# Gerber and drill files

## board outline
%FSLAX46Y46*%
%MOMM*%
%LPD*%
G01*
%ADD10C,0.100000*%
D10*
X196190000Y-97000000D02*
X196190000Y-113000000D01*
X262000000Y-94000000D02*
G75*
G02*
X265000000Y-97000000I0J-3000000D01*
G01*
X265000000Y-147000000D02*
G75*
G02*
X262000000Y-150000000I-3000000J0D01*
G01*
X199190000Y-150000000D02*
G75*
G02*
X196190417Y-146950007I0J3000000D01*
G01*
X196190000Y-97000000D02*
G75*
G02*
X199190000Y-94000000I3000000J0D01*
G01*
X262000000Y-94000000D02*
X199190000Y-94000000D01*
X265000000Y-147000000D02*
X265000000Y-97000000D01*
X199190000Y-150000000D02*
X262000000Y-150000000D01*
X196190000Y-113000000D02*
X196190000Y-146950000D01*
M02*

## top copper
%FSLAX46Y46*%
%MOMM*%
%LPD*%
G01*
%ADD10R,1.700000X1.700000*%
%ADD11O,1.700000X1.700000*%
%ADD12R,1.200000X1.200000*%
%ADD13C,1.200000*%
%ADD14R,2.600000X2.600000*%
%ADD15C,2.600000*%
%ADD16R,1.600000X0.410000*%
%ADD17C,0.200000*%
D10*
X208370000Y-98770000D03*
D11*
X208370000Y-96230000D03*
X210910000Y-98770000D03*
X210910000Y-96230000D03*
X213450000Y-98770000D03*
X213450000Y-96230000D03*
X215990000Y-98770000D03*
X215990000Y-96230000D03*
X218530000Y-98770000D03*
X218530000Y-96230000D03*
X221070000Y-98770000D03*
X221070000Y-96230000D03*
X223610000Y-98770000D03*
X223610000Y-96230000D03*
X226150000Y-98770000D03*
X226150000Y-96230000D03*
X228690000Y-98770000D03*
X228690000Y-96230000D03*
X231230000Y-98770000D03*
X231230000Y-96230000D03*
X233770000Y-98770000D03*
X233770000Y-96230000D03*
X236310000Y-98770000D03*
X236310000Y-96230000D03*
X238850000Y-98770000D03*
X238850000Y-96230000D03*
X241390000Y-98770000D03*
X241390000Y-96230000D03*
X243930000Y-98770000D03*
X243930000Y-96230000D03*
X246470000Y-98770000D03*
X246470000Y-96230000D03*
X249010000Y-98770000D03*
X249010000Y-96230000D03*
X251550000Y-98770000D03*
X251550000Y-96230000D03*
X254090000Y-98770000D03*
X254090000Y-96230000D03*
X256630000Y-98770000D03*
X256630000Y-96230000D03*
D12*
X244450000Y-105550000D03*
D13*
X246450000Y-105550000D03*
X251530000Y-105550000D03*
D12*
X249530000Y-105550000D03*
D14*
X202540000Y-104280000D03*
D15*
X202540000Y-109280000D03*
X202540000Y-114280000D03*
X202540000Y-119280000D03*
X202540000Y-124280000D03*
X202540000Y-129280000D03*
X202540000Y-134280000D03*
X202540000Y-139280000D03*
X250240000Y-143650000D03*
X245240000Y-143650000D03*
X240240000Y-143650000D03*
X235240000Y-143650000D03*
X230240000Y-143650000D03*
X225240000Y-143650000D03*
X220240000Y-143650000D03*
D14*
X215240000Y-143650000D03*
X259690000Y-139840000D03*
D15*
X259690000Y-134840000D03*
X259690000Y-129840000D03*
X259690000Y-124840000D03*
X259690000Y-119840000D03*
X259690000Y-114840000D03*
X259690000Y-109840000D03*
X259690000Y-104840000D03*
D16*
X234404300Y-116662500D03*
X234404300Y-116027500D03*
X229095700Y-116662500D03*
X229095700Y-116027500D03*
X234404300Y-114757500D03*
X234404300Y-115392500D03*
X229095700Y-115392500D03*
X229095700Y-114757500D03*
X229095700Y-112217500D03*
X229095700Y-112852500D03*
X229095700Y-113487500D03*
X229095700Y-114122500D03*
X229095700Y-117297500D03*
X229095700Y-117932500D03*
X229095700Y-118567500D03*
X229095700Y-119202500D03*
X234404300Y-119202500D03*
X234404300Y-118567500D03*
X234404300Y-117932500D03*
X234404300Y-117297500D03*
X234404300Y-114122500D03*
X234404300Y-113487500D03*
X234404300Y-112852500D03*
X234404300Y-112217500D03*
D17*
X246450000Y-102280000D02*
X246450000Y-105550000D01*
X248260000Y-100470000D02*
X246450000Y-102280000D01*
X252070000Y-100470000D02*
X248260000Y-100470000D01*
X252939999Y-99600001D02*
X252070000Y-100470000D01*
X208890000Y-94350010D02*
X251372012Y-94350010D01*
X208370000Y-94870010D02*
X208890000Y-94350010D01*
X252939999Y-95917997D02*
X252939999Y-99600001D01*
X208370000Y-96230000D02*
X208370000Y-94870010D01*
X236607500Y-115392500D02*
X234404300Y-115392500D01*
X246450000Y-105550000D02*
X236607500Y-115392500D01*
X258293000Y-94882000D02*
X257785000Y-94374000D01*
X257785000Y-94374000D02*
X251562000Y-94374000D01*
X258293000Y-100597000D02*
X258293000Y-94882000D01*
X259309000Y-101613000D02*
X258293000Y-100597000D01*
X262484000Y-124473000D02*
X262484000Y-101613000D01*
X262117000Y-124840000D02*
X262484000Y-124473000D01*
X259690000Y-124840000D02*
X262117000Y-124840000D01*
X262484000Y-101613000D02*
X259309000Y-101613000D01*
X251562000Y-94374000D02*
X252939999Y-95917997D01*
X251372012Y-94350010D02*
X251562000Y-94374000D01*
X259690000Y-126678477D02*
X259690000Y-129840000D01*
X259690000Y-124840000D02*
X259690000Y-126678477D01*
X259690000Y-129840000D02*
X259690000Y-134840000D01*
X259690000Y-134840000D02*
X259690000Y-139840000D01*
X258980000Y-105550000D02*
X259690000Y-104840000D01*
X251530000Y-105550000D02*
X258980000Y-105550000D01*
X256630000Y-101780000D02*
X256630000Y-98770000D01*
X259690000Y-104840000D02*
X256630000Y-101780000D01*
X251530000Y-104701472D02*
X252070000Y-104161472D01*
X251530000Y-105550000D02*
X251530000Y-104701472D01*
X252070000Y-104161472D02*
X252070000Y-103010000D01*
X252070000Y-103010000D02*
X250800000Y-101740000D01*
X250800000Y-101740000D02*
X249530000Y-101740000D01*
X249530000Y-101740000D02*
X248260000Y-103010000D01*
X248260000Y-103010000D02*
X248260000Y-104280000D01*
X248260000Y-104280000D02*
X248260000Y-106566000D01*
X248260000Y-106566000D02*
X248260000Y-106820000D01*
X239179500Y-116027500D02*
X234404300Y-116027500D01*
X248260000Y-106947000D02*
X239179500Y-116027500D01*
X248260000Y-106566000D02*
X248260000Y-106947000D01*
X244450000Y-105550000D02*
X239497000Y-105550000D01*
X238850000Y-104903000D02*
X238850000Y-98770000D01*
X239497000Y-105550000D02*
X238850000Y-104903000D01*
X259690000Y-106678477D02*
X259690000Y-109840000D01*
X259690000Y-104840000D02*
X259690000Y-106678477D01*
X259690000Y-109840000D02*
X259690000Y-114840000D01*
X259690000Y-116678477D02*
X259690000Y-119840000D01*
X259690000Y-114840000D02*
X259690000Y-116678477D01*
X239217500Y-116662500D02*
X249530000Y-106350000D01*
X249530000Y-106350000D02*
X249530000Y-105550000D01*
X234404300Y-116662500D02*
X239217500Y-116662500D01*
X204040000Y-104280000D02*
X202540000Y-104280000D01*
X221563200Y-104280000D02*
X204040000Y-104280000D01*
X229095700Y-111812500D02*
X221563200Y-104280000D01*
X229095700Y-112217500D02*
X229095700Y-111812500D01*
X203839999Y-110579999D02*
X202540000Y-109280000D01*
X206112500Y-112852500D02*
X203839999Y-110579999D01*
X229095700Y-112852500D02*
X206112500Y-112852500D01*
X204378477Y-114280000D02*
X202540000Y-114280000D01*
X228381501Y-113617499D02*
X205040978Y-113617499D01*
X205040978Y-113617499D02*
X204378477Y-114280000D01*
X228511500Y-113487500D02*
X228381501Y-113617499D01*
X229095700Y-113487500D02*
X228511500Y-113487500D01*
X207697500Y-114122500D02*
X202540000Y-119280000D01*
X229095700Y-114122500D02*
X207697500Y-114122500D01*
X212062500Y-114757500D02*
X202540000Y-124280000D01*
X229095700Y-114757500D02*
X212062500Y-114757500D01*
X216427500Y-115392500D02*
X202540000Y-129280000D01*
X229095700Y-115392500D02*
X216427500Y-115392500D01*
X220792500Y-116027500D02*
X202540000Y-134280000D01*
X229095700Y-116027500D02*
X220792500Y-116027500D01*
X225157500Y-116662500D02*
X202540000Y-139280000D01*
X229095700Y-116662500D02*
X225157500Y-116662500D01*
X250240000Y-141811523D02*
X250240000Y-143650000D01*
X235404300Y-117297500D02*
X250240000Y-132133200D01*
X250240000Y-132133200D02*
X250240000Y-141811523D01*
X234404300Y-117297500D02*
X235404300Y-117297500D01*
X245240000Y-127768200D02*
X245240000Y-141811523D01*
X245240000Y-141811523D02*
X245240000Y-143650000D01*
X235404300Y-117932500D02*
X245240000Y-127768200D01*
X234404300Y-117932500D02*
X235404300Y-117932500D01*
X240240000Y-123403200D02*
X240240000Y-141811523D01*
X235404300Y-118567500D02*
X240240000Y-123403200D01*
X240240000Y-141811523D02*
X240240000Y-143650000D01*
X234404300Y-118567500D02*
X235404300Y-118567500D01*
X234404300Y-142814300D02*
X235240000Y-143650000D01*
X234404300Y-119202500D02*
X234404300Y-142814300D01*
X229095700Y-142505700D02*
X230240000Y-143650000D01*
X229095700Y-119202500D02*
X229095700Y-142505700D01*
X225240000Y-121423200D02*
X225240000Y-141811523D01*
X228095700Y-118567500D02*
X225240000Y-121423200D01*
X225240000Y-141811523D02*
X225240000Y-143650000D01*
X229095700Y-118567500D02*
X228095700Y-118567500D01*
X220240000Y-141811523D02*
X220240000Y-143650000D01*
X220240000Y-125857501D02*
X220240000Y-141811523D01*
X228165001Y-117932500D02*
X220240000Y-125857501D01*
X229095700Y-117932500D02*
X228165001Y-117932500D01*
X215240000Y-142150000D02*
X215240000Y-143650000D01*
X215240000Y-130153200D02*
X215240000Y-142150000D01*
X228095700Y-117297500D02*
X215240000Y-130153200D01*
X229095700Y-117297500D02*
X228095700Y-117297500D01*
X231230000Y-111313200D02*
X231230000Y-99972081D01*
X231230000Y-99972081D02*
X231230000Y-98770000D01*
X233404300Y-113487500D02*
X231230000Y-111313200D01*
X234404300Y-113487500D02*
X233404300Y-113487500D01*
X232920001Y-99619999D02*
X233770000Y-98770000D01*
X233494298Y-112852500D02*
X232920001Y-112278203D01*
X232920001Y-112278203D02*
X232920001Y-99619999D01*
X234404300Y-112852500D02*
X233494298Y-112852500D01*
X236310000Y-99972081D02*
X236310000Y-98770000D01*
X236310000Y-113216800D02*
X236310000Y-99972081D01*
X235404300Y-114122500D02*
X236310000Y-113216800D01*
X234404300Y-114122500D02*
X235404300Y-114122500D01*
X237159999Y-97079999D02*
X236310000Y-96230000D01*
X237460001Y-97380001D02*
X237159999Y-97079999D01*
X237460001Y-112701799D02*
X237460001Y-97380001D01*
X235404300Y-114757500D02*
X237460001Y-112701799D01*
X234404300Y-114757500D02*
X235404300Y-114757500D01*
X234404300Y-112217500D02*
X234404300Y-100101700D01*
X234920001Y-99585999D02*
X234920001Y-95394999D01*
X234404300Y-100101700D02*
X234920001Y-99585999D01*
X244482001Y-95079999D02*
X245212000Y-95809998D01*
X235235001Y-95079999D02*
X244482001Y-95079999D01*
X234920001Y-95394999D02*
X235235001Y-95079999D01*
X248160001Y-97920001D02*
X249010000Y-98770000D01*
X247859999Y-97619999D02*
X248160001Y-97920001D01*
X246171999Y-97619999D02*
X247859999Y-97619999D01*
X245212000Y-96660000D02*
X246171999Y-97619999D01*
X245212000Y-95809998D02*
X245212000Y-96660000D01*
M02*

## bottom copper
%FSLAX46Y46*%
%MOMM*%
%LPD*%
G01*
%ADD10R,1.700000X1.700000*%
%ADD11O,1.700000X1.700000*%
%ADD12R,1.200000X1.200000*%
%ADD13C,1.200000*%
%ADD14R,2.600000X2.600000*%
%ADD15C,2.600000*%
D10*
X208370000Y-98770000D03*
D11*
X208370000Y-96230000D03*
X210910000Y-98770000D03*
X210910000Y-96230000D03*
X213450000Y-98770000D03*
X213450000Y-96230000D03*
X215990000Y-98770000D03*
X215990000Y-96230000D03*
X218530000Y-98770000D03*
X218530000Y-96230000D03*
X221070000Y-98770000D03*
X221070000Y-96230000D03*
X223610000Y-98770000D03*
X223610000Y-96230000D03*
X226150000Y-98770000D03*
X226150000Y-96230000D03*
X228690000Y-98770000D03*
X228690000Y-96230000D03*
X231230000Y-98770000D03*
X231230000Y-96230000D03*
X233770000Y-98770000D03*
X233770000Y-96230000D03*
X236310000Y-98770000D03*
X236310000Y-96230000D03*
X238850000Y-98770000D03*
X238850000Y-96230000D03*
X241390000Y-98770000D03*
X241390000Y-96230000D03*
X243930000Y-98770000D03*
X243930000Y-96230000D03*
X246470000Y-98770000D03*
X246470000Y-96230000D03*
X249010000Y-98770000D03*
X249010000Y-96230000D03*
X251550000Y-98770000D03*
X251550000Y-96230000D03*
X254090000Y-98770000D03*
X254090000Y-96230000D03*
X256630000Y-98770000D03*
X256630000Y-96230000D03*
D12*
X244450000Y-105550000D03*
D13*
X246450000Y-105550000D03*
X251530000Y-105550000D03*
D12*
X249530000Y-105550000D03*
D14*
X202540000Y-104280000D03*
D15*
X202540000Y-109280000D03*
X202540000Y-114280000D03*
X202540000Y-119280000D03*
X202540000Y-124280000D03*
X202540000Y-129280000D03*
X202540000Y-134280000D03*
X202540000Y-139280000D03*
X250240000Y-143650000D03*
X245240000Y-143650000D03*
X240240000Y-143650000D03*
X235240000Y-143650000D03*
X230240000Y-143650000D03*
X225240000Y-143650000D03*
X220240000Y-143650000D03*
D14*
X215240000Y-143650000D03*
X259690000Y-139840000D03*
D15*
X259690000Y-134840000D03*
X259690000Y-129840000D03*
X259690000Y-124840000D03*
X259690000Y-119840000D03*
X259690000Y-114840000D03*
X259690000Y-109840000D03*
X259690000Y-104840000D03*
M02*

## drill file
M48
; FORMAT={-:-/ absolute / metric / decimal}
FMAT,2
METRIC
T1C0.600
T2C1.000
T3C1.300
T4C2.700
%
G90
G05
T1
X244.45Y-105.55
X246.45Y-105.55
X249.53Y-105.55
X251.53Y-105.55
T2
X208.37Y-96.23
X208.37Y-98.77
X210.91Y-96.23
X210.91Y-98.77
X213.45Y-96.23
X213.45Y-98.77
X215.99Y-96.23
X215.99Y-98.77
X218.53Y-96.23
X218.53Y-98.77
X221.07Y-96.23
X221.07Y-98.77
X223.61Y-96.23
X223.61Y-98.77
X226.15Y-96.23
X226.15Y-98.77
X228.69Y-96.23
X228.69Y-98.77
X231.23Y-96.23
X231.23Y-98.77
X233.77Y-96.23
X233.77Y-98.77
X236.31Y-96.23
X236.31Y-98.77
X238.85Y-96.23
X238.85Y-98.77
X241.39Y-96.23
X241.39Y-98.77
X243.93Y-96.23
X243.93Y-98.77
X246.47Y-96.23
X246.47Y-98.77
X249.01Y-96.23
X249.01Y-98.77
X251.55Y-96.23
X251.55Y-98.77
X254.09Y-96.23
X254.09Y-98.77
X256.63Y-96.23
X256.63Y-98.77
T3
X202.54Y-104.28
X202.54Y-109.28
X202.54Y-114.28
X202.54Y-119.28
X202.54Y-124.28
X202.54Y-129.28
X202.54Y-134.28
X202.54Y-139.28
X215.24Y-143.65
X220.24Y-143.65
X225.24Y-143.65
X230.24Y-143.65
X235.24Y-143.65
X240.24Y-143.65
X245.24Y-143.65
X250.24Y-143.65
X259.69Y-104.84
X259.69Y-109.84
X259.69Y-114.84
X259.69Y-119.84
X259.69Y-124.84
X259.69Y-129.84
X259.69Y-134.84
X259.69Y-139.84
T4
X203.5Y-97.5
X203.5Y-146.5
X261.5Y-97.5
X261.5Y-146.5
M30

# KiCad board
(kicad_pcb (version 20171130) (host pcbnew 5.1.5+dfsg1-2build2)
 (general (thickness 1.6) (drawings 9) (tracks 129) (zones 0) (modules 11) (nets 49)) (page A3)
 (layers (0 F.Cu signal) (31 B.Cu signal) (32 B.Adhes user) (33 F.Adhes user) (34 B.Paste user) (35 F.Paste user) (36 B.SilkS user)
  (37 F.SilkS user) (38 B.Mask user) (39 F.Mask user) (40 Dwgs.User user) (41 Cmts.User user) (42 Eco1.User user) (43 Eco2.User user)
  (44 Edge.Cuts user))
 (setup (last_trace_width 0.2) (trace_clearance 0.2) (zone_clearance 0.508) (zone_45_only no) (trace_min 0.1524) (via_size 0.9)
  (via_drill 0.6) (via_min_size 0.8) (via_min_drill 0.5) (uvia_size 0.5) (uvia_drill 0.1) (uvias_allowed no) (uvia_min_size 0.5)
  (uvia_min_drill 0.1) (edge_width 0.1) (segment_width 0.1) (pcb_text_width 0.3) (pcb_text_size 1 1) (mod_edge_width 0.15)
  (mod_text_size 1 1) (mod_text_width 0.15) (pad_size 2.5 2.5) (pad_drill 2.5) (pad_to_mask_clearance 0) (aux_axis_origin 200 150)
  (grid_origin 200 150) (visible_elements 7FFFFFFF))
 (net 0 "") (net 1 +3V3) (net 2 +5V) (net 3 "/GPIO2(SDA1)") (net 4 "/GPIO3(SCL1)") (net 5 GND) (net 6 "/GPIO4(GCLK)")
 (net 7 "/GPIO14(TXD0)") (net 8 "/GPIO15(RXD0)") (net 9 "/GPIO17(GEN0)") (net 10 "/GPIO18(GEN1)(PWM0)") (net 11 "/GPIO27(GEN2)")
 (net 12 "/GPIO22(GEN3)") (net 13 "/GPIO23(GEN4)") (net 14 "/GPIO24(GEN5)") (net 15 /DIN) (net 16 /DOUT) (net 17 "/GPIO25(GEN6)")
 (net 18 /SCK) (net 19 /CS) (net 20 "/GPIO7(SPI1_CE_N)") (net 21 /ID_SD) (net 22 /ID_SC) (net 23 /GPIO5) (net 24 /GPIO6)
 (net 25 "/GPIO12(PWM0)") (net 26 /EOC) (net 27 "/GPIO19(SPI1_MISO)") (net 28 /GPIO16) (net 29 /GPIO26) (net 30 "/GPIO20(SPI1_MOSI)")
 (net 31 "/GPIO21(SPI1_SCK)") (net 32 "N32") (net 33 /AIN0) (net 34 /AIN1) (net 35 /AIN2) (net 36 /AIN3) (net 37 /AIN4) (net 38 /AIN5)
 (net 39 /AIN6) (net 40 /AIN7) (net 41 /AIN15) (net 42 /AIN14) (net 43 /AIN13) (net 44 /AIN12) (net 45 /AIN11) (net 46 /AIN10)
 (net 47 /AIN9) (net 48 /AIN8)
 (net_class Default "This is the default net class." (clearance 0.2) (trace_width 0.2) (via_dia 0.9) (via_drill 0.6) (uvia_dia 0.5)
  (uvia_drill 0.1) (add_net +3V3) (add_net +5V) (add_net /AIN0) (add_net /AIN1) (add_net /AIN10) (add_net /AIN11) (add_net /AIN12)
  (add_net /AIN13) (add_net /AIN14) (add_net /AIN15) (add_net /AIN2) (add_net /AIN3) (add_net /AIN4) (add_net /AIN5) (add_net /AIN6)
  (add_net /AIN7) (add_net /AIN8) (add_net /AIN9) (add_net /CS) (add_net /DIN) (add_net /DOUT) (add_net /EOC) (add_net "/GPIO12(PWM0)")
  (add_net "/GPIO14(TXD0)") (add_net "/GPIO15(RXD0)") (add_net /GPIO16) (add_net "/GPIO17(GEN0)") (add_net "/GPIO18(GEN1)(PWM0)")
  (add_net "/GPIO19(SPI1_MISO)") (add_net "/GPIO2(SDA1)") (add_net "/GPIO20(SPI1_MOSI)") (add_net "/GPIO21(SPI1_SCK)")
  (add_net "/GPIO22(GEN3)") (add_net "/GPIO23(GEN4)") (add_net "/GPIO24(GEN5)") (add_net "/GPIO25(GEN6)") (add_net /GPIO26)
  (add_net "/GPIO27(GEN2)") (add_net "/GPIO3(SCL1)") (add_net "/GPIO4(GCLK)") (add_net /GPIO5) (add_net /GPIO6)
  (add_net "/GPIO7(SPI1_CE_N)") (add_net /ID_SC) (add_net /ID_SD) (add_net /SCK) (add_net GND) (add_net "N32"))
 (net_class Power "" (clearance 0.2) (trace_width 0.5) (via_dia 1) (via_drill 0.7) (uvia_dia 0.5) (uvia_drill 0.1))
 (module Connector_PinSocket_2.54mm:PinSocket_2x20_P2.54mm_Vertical (layer B.Cu) (at 208.37 98.77 270)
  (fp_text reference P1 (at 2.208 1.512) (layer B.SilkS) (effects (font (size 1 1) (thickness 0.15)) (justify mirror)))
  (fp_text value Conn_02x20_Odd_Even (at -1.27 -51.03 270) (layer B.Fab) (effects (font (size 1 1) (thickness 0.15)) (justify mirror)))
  (pad 1 thru_hole rect (at 0 0 270) (size 1.7 1.7) (drill 1) (layers *.Cu *.Mask) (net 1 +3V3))
  (pad 2 thru_hole oval (at -2.54 0 270) (size 1.7 1.7) (drill 1) (layers *.Cu *.Mask) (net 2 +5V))
  (pad 3 thru_hole oval (at 0 -2.54 270) (size 1.7 1.7) (drill 1) (layers *.Cu *.Mask) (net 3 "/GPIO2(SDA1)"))
  (pad 4 thru_hole oval (at -2.54 -2.54 270) (size 1.7 1.7) (drill 1) (layers *.Cu *.Mask) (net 2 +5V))
  (pad 5 thru_hole oval (at 0 -5.08 270) (size 1.7 1.7) (drill 1) (layers *.Cu *.Mask) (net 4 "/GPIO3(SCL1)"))
  (pad 6 thru_hole oval (at -2.54 -5.08 270) (size 1.7 1.7) (drill 1) (layers *.Cu *.Mask) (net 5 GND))
  (pad 7 thru_hole oval (at 0 -7.62 270) (size 1.7 1.7) (drill 1) (layers *.Cu *.Mask) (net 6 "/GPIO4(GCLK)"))
  (pad 8 thru_hole oval (at -2.54 -7.62 270) (size 1.7 1.7) (drill 1) (layers *.Cu *.Mask) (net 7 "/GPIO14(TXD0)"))
  (pad 9 thru_hole oval (at 0 -10.16 270) (size 1.7 1.7) (drill 1) (layers *.Cu *.Mask) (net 5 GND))
  (pad 10 thru_hole oval (at -2.54 -10.16 270) (size 1.7 1.7) (drill 1) (layers *.Cu *.Mask) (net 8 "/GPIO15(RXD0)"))
  (pad 11 thru_hole oval (at 0 -12.7 270) (size 1.7 1.7) (drill 1) (layers *.Cu *.Mask) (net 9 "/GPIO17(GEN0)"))
  (pad 12 thru_hole oval (at -2.54 -12.7 270) (size 1.7 1.7) (drill 1) (layers *.Cu *.Mask) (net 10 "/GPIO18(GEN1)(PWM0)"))
  (pad 13 thru_hole oval (at 0 -15.24 270) (size 1.7 1.7) (drill 1) (layers *.Cu *.Mask) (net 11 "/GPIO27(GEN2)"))
  (pad 14 thru_hole oval (at -2.54 -15.24 270) (size 1.7 1.7) (drill 1) (layers *.Cu *.Mask) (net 5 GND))
  (pad 15 thru_hole oval (at 0 -17.78 270) (size 1.7 1.7) (drill 1) (layers *.Cu *.Mask) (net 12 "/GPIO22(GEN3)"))
  (pad 16 thru_hole oval (at -2.54 -17.78 270) (size 1.7 1.7) (drill 1) (layers *.Cu *.Mask) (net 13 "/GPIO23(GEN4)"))
  (pad 17 thru_hole oval (at 0 -20.32 270) (size 1.7 1.7) (drill 1) (layers *.Cu *.Mask) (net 1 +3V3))
  (pad 18 thru_hole oval (at -2.54 -20.32 270) (size 1.7 1.7) (drill 1) (layers *.Cu *.Mask) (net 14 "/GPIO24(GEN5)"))
  (pad 19 thru_hole oval (at 0 -22.86 270) (size 1.7 1.7) (drill 1) (layers *.Cu *.Mask) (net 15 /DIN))
  (pad 20 thru_hole oval (at -2.54 -22.86 270) (size 1.7 1.7) (drill 1) (layers *.Cu *.Mask) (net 5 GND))
  (pad 21 thru_hole oval (at 0 -25.4 270) (size 1.7 1.7) (drill 1) (layers *.Cu *.Mask) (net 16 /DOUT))
  (pad 22 thru_hole oval (at -2.54 -25.4 270) (size 1.7 1.7) (drill 1) (layers *.Cu *.Mask) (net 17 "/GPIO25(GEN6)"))
  (pad 23 thru_hole oval (at 0 -27.94 270) (size 1.7 1.7) (drill 1) (layers *.Cu *.Mask) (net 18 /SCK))
  (pad 24 thru_hole oval (at -2.54 -27.94 270) (size 1.7 1.7) (drill 1) (layers *.Cu *.Mask) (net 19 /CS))
  (pad 25 thru_hole oval (at 0 -30.48 270) (size 1.7 1.7) (drill 1) (layers *.Cu *.Mask) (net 5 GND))
  (pad 26 thru_hole oval (at -2.54 -30.48 270) (size 1.7 1.7) (drill 1) (layers *.Cu *.Mask) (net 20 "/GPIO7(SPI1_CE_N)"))
  (pad 27 thru_hole oval (at 0 -33.02 270) (size 1.7 1.7) (drill 1) (layers *.Cu *.Mask) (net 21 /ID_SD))
  (pad 28 thru_hole oval (at -2.54 -33.02 270) (size 1.7 1.7) (drill 1) (layers *.Cu *.Mask) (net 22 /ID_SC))
  (pad 29 thru_hole oval (at 0 -35.56 270) (size 1.7 1.7) (drill 1) (layers *.Cu *.Mask) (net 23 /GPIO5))
  (pad 30 thru_hole oval (at -2.54 -35.56 270) (size 1.7 1.7) (drill 1) (layers *.Cu *.Mask) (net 5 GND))
  (pad 31 thru_hole oval (at 0 -38.1 270) (size 1.7 1.7) (drill 1) (layers *.Cu *.Mask) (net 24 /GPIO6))
  (pad 32 thru_hole oval (at -2.54 -38.1 270) (size 1.7 1.7) (drill 1) (layers *.Cu *.Mask) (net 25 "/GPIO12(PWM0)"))
  (pad 33 thru_hole oval (at 0 -40.64 270) (size 1.7 1.7) (drill 1) (layers *.Cu *.Mask) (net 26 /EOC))
  (pad 34 thru_hole oval (at -2.54 -40.64 270) (size 1.7 1.7) (drill 1) (layers *.Cu *.Mask) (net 5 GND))
  (pad 35 thru_hole oval (at 0 -43.18 270) (size 1.7 1.7) (drill 1) (layers *.Cu *.Mask) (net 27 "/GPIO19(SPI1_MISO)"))
  (pad 36 thru_hole oval (at -2.54 -43.18 270) (size 1.7 1.7) (drill 1) (layers *.Cu *.Mask) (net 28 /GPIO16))
  (pad 37 thru_hole oval (at 0 -45.72 270) (size 1.7 1.7) (drill 1) (layers *.Cu *.Mask) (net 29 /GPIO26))
  (pad 38 thru_hole oval (at -2.54 -45.72 270) (size 1.7 1.7) (drill 1) (layers *.Cu *.Mask) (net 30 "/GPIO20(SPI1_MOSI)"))
  (pad 39 thru_hole oval (at 0 -48.26 270) (size 1.7 1.7) (drill 1) (layers *.Cu *.Mask) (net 5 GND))
  (pad 40 thru_hole oval (at -2.54 -48.26 270) (size 1.7 1.7) (drill 1) (layers *.Cu *.Mask) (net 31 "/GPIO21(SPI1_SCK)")))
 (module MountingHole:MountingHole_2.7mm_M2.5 (layer F.Cu) (at 261.5 146.5)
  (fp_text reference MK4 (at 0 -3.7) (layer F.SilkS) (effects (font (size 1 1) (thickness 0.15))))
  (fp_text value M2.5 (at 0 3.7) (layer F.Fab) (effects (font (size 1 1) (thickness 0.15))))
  (pad 1 np_thru_hole circle (at 0 0) (size 2.7 2.7) (drill 2.7) (layers *.Cu *.Mask)))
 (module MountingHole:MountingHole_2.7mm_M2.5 (layer F.Cu) (at 203.5 146.5)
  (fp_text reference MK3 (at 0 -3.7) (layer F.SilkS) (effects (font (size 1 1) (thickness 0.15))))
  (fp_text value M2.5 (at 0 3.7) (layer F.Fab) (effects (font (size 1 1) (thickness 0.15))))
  (pad 1 np_thru_hole circle (at 0 0) (size 2.7 2.7) (drill 2.7) (layers *.Cu *.Mask)))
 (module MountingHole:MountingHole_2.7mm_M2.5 (layer F.Cu) (at 261.5 97.5 180)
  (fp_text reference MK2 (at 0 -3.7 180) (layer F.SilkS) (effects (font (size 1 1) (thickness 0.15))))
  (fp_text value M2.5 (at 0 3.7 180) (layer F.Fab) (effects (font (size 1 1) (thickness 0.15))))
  (pad 1 np_thru_hole circle (at 0 0 180) (size 2.7 2.7) (drill 2.7) (layers *.Cu *.Mask)))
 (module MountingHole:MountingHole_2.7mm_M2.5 (layer F.Cu) (at 203.5 97.5 180)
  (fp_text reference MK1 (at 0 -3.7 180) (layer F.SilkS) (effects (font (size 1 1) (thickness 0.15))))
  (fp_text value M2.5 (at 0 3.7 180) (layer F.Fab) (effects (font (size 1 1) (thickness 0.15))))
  (pad 1 np_thru_hole circle (at 0 0 180) (size 2.7 2.7) (drill 2.7) (layers *.Cu *.Mask)))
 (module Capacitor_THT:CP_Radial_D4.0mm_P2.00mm (layer F.Cu) (at 244.45 105.55)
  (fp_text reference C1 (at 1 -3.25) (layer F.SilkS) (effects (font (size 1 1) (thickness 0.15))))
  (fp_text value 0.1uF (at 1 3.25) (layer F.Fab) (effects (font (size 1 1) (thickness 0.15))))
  (pad 1 thru_hole rect (at 0 0) (size 1.2 1.2) (drill 0.6) (layers *.Cu *.Mask) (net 5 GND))
  (pad 2 thru_hole circle (at 2 0) (size 1.2 1.2) (drill 0.6) (layers *.Cu *.Mask) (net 2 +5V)))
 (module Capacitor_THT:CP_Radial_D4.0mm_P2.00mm (layer F.Cu) (at 249.53 105.55)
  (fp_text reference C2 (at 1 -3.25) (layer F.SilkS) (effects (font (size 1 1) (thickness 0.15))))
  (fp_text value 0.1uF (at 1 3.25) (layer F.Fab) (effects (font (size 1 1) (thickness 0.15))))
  (pad 2 thru_hole circle (at 2 0) (size 1.2 1.2) (drill 0.6) (layers *.Cu *.Mask) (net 5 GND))
  (pad 1 thru_hole rect (at 0 0) (size 1.2 1.2) (drill 0.6) (layers *.Cu *.Mask) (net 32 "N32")))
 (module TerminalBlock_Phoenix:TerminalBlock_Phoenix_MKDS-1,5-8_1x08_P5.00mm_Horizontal (layer F.Cu) (at 202.54 104.28 270)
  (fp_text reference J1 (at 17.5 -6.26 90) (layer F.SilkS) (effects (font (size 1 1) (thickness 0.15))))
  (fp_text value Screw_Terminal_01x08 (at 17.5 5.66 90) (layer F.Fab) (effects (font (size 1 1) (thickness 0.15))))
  (pad 1 thru_hole rect (at 0 0 270) (size 2.6 2.6) (drill 1.3) (layers *.Cu *.Mask) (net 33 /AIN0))
  (pad 2 thru_hole circle (at 5 0 270) (size 2.6 2.6) (drill 1.3) (layers *.Cu *.Mask) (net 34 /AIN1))
  (pad 3 thru_hole circle (at 10 0 270) (size 2.6 2.6) (drill 1.3) (layers *.Cu *.Mask) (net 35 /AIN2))
  (pad 4 thru_hole circle (at 15 0 270) (size 2.6 2.6) (drill 1.3) (layers *.Cu *.Mask) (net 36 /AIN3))
  (pad 5 thru_hole circle (at 20 0 270) (size 2.6 2.6) (drill 1.3) (layers *.Cu *.Mask) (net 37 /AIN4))
  (pad 6 thru_hole circle (at 25 0 270) (size 2.6 2.6) (drill 1.3) (layers *.Cu *.Mask) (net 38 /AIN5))
  (pad 7 thru_hole circle (at 30 0 270) (size 2.6 2.6) (drill 1.3) (layers *.Cu *.Mask) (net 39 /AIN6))
  (pad 8 thru_hole circle (at 35 0 270) (size 2.6 2.6) (drill 1.3) (layers *.Cu *.Mask) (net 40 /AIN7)))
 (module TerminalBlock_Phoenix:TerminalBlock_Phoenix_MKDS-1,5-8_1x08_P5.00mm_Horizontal (layer F.Cu) (at 215.24 143.65)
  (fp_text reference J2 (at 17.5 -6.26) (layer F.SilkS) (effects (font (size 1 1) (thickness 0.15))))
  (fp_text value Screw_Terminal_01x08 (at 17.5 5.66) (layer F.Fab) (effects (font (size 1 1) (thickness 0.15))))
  (pad 8 thru_hole circle (at 35 0) (size 2.6 2.6) (drill 1.3) (layers *.Cu *.Mask) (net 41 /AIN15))
  (pad 7 thru_hole circle (at 30 0) (size 2.6 2.6) (drill 1.3) (layers *.Cu *.Mask) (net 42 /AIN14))
  (pad 6 thru_hole circle (at 25 0) (size 2.6 2.6) (drill 1.3) (layers *.Cu *.Mask) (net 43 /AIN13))
  (pad 5 thru_hole circle (at 20 0) (size 2.6 2.6) (drill 1.3) (layers *.Cu *.Mask) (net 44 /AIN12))
  (pad 4 thru_hole circle (at 15 0) (size 2.6 2.6) (drill 1.3) (layers *.Cu *.Mask) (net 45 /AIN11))
  (pad 3 thru_hole circle (at 10 0) (size 2.6 2.6) (drill 1.3) (layers *.Cu *.Mask) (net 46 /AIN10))
  (pad 2 thru_hole circle (at 5 0) (size 2.6 2.6) (drill 1.3) (layers *.Cu *.Mask) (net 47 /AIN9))
  (pad 1 thru_hole rect (at 0 0) (size 2.6 2.6) (drill 1.3) (layers *.Cu *.Mask) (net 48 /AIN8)))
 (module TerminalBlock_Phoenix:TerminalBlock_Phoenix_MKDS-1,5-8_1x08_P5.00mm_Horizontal (layer F.Cu) (at 259.69 139.84 90)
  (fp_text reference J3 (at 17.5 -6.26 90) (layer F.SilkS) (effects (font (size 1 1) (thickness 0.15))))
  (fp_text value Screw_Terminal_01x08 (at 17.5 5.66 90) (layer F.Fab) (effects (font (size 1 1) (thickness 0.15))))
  (pad 1 thru_hole rect (at 0 0 90) (size 2.6 2.6) (drill 1.3) (layers *.Cu *.Mask) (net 2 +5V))
  (pad 2 thru_hole circle (at 5 0 90) (size 2.6 2.6) (drill 1.3) (layers *.Cu *.Mask) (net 2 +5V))
  (pad 3 thru_hole circle (at 10 0 90) (size 2.6 2.6) (drill 1.3) (layers *.Cu *.Mask) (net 2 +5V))
  (pad 4 thru_hole circle (at 15 0 90) (size 2.6 2.6) (drill 1.3) (layers *.Cu *.Mask) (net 2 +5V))
  (pad 5 thru_hole circle (at 20 0 90) (size 2.6 2.6) (drill 1.3) (layers *.Cu *.Mask) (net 5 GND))
  (pad 6 thru_hole circle (at 25 0 90) (size 2.6 2.6) (drill 1.3) (layers *.Cu *.Mask) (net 5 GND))
  (pad 7 thru_hole circle (at 30 0 90) (size 2.6 2.6) (drill 1.3) (layers *.Cu *.Mask) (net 5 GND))
  (pad 8 thru_hole circle (at 35 0 90) (size 2.6 2.6) (drill 1.3) (layers *.Cu *.Mask) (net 5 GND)))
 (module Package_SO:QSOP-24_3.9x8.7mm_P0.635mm (layer F.Cu) (at 231.75 115.71)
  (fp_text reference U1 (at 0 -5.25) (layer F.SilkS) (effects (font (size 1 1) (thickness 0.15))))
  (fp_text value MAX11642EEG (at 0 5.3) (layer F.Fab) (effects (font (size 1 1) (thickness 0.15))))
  (pad 17 smd rect (at 2.6543 0.9525) (size 1.6 0.41) (layers F.Cu F.Paste F.Mask) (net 32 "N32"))
  (pad 18 smd rect (at 2.6543 0.3175) (size 1.6 0.41) (layers F.Cu F.Paste F.Mask) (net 5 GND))
  (pad 8 smd rect (at -2.6543 0.9525) (size 1.6 0.41) (layers F.Cu F.Paste F.Mask) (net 40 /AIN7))
  (pad 7 smd rect (at -2.6543 0.3175) (size 1.6 0.41) (layers F.Cu F.Paste F.Mask) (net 39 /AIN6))
  (pad 20 smd rect (at 2.6543 -0.9525) (size 1.6 0.41) (layers F.Cu F.Paste F.Mask) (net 19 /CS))
  (pad 19 smd rect (at 2.6543 -0.3175) (size 1.6 0.41) (layers F.Cu F.Paste F.Mask) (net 2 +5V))
  (pad 6 smd rect (at -2.6543 -0.3175) (size 1.6 0.41) (layers F.Cu F.Paste F.Mask) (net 38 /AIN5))
  (pad 5 smd rect (at -2.6543 -0.9525) (size 1.6 0.41) (layers F.Cu F.Paste F.Mask) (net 37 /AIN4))
  (pad 1 smd rect (at -2.6543 -3.4925) (size 1.6 0.41) (layers F.Cu F.Paste F.Mask) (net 33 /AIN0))
  (pad 2 smd rect (at -2.6543 -2.8575) (size 1.6 0.41) (layers F.Cu F.Paste F.Mask) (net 34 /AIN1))
  (pad 3 smd rect (at -2.6543 -2.2225) (size 1.6 0.41) (layers F.Cu F.Paste F.Mask) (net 35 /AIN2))
  (pad 4 smd rect (at -2.6543 -1.5875) (size 1.6 0.41) (layers F.Cu F.Paste F.Mask) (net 36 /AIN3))
  (pad 9 smd rect (at -2.6543 1.5875) (size 1.6 0.41) (layers F.Cu F.Paste F.Mask) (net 48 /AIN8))
  (pad 10 smd rect (at -2.6543 2.2225) (size 1.6 0.41) (layers F.Cu F.Paste F.Mask) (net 47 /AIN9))
  (pad 11 smd rect (at -2.6543 2.8575) (size 1.6 0.41) (layers F.Cu F.Paste F.Mask) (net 46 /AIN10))
  (pad 12 smd rect (at -2.6543 3.4925) (size 1.6 0.41) (layers F.Cu F.Paste F.Mask) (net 45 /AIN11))
  (pad 13 smd rect (at 2.6543 3.4925) (size 1.6 0.41) (layers F.Cu F.Paste F.Mask) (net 44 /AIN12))
  (pad 14 smd rect (at 2.6543 2.8575) (size 1.6 0.41) (layers F.Cu F.Paste F.Mask) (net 43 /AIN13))
  (pad 15 smd rect (at 2.6543 2.2225) (size 1.6 0.41) (layers F.Cu F.Paste F.Mask) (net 42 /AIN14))
  (pad 16 smd rect (at 2.6543 1.5875) (size 1.6 0.41) (layers F.Cu F.Paste F.Mask) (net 41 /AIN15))
  (pad 21 smd rect (at 2.6543 -1.5875) (size 1.6 0.41) (layers F.Cu F.Paste F.Mask) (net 18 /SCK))
  (pad 22 smd rect (at 2.6543 -2.2225) (size 1.6 0.41) (layers F.Cu F.Paste F.Mask) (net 15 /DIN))
  (pad 23 smd rect (at 2.6543 -2.8575) (size 1.6 0.41) (layers F.Cu F.Paste F.Mask) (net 16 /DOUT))
  (pad 24 smd rect (at 2.6543 -3.4925) (size 1.6 0.41) (layers F.Cu F.Paste F.Mask) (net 26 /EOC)))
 (gr_line (start 196.19 97) (end 196.19 113) (layer Edge.Cuts) (width 0.1))
 (gr_arc (start 262 97) (end 262 94) (angle 90) (layer Edge.Cuts) (width 0.1))
 (gr_arc (start 262 147) (end 265 147) (angle 90) (layer Edge.Cuts) (width 0.1))
 (gr_arc (start 199.19 147) (end 199.19 150) (angle 90.95484125) (layer Edge.Cuts) (width 0.1))
 (gr_arc (start 199.19 97) (end 196.19 97) (angle 90) (layer Edge.Cuts) (width 0.1))
 (gr_line (start 262 94) (end 199.19 94) (layer Edge.Cuts) (width 0.1))
 (gr_line (start 265 147) (end 265 97) (layer Edge.Cuts) (width 0.1))
 (gr_line (start 199.19 150) (end 262 150) (layer Edge.Cuts) (width 0.1))
 (gr_line (start 196.19 113) (end 196.19 146.95) (layer Edge.Cuts) (width 0.1))
 (segment (start 246.45 102.28) (end 246.45 105.55) (width 0.2) (layer F.Cu) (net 2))
 (segment (start 248.26 100.47) (end 246.45 102.28) (width 0.2) (layer F.Cu) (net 2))
 (segment (start 252.07 100.47) (end 248.26 100.47) (width 0.2) (layer F.Cu) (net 2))
 (segment (start 252.939999 99.600001) (end 252.07 100.47) (width 0.2) (layer F.Cu) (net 2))
 (segment (start 208.89 94.35001) (end 251.372012 94.35001) (width 0.2) (layer F.Cu) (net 2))
 (segment (start 208.37 94.87001) (end 208.89 94.35001) (width 0.2) (layer F.Cu) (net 2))
 (segment (start 252.939999 95.917997) (end 252.939999 99.600001) (width 0.2) (layer F.Cu) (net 2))
 (segment (start 208.37 96.23) (end 208.37 94.87001) (width 0.2) (layer F.Cu) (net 2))
 (segment (start 236.6075 115.3925) (end 234.4043 115.3925) (width 0.2) (layer F.Cu) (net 2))
 (segment (start 246.45 105.55) (end 236.6075 115.3925) (width 0.2) (layer F.Cu) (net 2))
 (segment (start 258.293 94.882) (end 257.785 94.374) (width 0.2) (layer F.Cu) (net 2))
 (segment (start 257.785 94.374) (end 251.562 94.374) (width 0.2) (layer F.Cu) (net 2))
 (segment (start 258.293 100.597) (end 258.293 94.882) (width 0.2) (layer F.Cu) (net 2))
 (segment (start 259.309 101.613) (end 258.293 100.597) (width 0.2) (layer F.Cu) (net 2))
 (segment (start 262.484 124.473) (end 262.484 101.613) (width 0.2) (layer F.Cu) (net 2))
 (segment (start 262.117 124.84) (end 262.484 124.473) (width 0.2) (layer F.Cu) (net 2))
 (segment (start 259.69 124.84) (end 262.117 124.84) (width 0.2) (layer F.Cu) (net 2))
 (segment (start 262.484 101.613) (end 259.309 101.613) (width 0.2) (layer F.Cu) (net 2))
 (segment (start 251.562 94.374) (end 252.939999 95.917997) (width 0.2) (layer F.Cu) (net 2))
 (segment (start 251.372012 94.35001) (end 251.562 94.374) (width 0.2) (layer F.Cu) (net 2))
 (segment (start 259.69 126.678477) (end 259.69 129.84) (width 0.2) (layer F.Cu) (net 2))
 (segment (start 259.69 124.84) (end 259.69 126.678477) (width 0.2) (layer F.Cu) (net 2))
 (segment (start 259.69 129.84) (end 259.69 134.84) (width 0.2) (layer F.Cu) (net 2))
 (segment (start 259.69 134.84) (end 259.69 139.84) (width 0.2) (layer F.Cu) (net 2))
 (segment (start 258.98 105.55) (end 259.69 104.84) (width 0.2) (layer F.Cu) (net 5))
 (segment (start 251.53 105.55) (end 258.98 105.55) (width 0.2) (layer F.Cu) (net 5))
 (segment (start 256.63 101.78) (end 256.63 98.77) (width 0.2) (layer F.Cu) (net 5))
 (segment (start 259.69 104.84) (end 256.63 101.78) (width 0.2) (layer F.Cu) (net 5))
 (segment (start 251.53 104.701472) (end 252.07 104.161472) (width 0.2) (layer F.Cu) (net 5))
 (segment (start 251.53 105.55) (end 251.53 104.701472) (width 0.2) (layer F.Cu) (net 5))
 (segment (start 252.07 104.161472) (end 252.07 103.01) (width 0.2) (layer F.Cu) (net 5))
 (segment (start 252.07 103.01) (end 250.8 101.74) (width 0.2) (layer F.Cu) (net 5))
 (segment (start 250.8 101.74) (end 249.53 101.74) (width 0.2) (layer F.Cu) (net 5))
 (segment (start 249.53 101.74) (end 248.26 103.01) (width 0.2) (layer F.Cu) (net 5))
 (segment (start 248.26 103.01) (end 248.26 104.28) (width 0.2) (layer F.Cu) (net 5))
 (segment (start 248.26 104.28) (end 248.26 106.566) (width 0.2) (layer F.Cu) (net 5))
 (segment (start 248.26 106.566) (end 248.26 106.82) (width 0.2) (layer F.Cu) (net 5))
 (segment (start 239.1795 116.0275) (end 234.4043 116.0275) (width 0.2) (layer F.Cu) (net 5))
 (segment (start 248.26 106.947) (end 239.1795 116.0275) (width 0.2) (layer F.Cu) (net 5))
 (segment (start 248.26 106.566) (end 248.26 106.947) (width 0.2) (layer F.Cu) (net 5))
 (segment (start 244.45 105.55) (end 239.497 105.55) (width 0.2) (layer F.Cu) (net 5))
 (segment (start 238.85 104.903) (end 238.85 98.77) (width 0.2) (layer F.Cu) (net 5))
 (segment (start 239.497 105.55) (end 238.85 104.903) (width 0.2) (layer F.Cu) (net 5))
 (segment (start 259.69 106.678477) (end 259.69 109.84) (width 0.2) (layer F.Cu) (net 5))
 (segment (start 259.69 104.84) (end 259.69 106.678477) (width 0.2) (layer F.Cu) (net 5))
 (segment (start 259.69 109.84) (end 259.69 114.84) (width 0.2) (layer F.Cu) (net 5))
 (segment (start 259.69 116.678477) (end 259.69 119.84) (width 0.2) (layer F.Cu) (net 5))
 (segment (start 259.69 114.84) (end 259.69 116.678477) (width 0.2) (layer F.Cu) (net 5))
 (segment (start 239.2175 116.6625) (end 249.53 106.35) (width 0.2) (layer F.Cu) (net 32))
 (segment (start 249.53 106.35) (end 249.53 105.55) (width 0.2) (layer F.Cu) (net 32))
 (segment (start 234.4043 116.6625) (end 239.2175 116.6625) (width 0.2) (layer F.Cu) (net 32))
 (segment (start 204.04 104.28) (end 202.54 104.28) (width 0.2) (layer F.Cu) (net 33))
 (segment (start 221.5632 104.28) (end 204.04 104.28) (width 0.2) (layer F.Cu) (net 33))
 (segment (start 229.0957 111.8125) (end 221.5632 104.28) (width 0.2) (layer F.Cu) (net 33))
 (segment (start 229.0957 112.2175) (end 229.0957 111.8125) (width 0.2) (layer F.Cu) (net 33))
 (segment (start 203.839999 110.579999) (end 202.54 109.28) (width 0.2) (layer F.Cu) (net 34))
 (segment (start 206.1125 112.8525) (end 203.839999 110.579999) (width 0.2) (layer F.Cu) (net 34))
 (segment (start 229.0957 112.8525) (end 206.1125 112.8525) (width 0.2) (layer F.Cu) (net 34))
 (segment (start 204.378477 114.28) (end 202.54 114.28) (width 0.2) (layer F.Cu) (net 35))
 (segment (start 228.381501 113.617499) (end 205.040978 113.617499) (width 0.2) (layer F.Cu) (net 35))
 (segment (start 205.040978 113.617499) (end 204.378477 114.28) (width 0.2) (layer F.Cu) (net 35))
 (segment (start 228.5115 113.4875) (end 228.381501 113.617499) (width 0.2) (layer F.Cu) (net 35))
 (segment (start 229.0957 113.4875) (end 228.5115 113.4875) (width 0.2) (layer F.Cu) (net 35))
 (segment (start 207.6975 114.1225) (end 202.54 119.28) (width 0.2) (layer F.Cu) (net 36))
 (segment (start 229.0957 114.1225) (end 207.6975 114.1225) (width 0.2) (layer F.Cu) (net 36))
 (segment (start 212.0625 114.7575) (end 202.54 124.28) (width 0.2) (layer F.Cu) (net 37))
 (segment (start 229.0957 114.7575) (end 212.0625 114.7575) (width 0.2) (layer F.Cu) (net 37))
 (segment (start 216.4275 115.3925) (end 202.54 129.28) (width 0.2) (layer F.Cu) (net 38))
 (segment (start 229.0957 115.3925) (end 216.4275 115.3925) (width 0.2) (layer F.Cu) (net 38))
 (segment (start 220.7925 116.0275) (end 202.54 134.28) (width 0.2) (layer F.Cu) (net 39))
 (segment (start 229.0957 116.0275) (end 220.7925 116.0275) (width 0.2) (layer F.Cu) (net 39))
 (segment (start 225.1575 116.6625) (end 202.54 139.28) (width 0.2) (layer F.Cu) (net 40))
 (segment (start 229.0957 116.6625) (end 225.1575 116.6625) (width 0.2) (layer F.Cu) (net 40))
 (segment (start 250.24 141.811523) (end 250.24 143.65) (width 0.2) (layer F.Cu) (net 41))
 (segment (start 235.4043 117.2975) (end 250.24 132.1332) (width 0.2) (layer F.Cu) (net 41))
 (segment (start 250.24 132.1332) (end 250.24 141.811523) (width 0.2) (layer F.Cu) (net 41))
 (segment (start 234.4043 117.2975) (end 235.4043 117.2975) (width 0.2) (layer F.Cu) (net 41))
 (segment (start 245.24 127.7682) (end 245.24 141.811523) (width 0.2) (layer F.Cu) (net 42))
 (segment (start 245.24 141.811523) (end 245.24 143.65) (width 0.2) (layer F.Cu) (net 42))
 (segment (start 235.4043 117.9325) (end 245.24 127.7682) (width 0.2) (layer F.Cu) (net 42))
 (segment (start 234.4043 117.9325) (end 235.4043 117.9325) (width 0.2) (layer F.Cu) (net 42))
 (segment (start 240.24 123.4032) (end 240.24 141.811523) (width 0.2) (layer F.Cu) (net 43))
 (segment (start 235.4043 118.5675) (end 240.24 123.4032) (width 0.2) (layer F.Cu) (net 43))
 (segment (start 240.24 141.811523) (end 240.24 143.65) (width 0.2) (layer F.Cu) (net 43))
 (segment (start 234.4043 118.5675) (end 235.4043 118.5675) (width 0.2) (layer F.Cu) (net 43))
 (segment (start 234.4043 142.8143) (end 235.24 143.65) (width 0.2) (layer F.Cu) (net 44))
 (segment (start 234.4043 119.2025) (end 234.4043 142.8143) (width 0.2) (layer F.Cu) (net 44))
 (segment (start 229.0957 142.5057) (end 230.24 143.65) (width 0.2) (layer F.Cu) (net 45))
 (segment (start 229.0957 119.2025) (end 229.0957 142.5057) (width 0.2) (layer F.Cu) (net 45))
 (segment (start 225.24 121.4232) (end 225.24 141.811523) (width 0.2) (layer F.Cu) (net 46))
 (segment (start 228.0957 118.5675) (end 225.24 121.4232) (width 0.2) (layer F.Cu) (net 46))
 (segment (start 225.24 141.811523) (end 225.24 143.65) (width 0.2) (layer F.Cu) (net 46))
 (segment (start 229.0957 118.5675) (end 228.0957 118.5675) (width 0.2) (layer F.Cu) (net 46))
 (segment (start 220.24 141.811523) (end 220.24 143.65) (width 0.2) (layer F.Cu) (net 47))
 (segment (start 220.24 125.857501) (end 220.24 141.811523) (width 0.2) (layer F.Cu) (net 47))
 (segment (start 228.165001 117.9325) (end 220.24 125.857501) (width 0.2) (layer F.Cu) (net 47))
 (segment (start 229.0957 117.9325) (end 228.165001 117.9325) (width 0.2) (layer F.Cu) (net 47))
 (segment (start 215.24 142.15) (end 215.24 143.65) (width 0.2) (layer F.Cu) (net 48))
 (segment (start 215.24 130.1532) (end 215.24 142.15) (width 0.2) (layer F.Cu) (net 48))
 (segment (start 228.0957 117.2975) (end 215.24 130.1532) (width 0.2) (layer F.Cu) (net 48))
 (segment (start 229.0957 117.2975) (end 228.0957 117.2975) (width 0.2) (layer F.Cu) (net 48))
 (segment (start 231.23 111.3132) (end 231.23 99.972081) (width 0.2) (layer F.Cu) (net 15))
 (segment (start 231.23 99.972081) (end 231.23 98.77) (width 0.2) (layer F.Cu) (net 15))
 (segment (start 233.4043 113.4875) (end 231.23 111.3132) (width 0.2) (layer F.Cu) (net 15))
 (segment (start 234.4043 113.4875) (end 233.4043 113.4875) (width 0.2) (layer F.Cu) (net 15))
 (segment (start 232.920001 99.619999) (end 233.77 98.77) (width 0.2) (layer F.Cu) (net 16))
 (segment (start 233.494298 112.8525) (end 232.920001 112.278203) (width 0.2) (layer F.Cu) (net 16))
 (segment (start 232.920001 112.278203) (end 232.920001 99.619999) (width 0.2) (layer F.Cu) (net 16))
 (segment (start 234.4043 112.8525) (end 233.494298 112.8525) (width 0.2) (layer F.Cu) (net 16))
 (segment (start 236.31 99.972081) (end 236.31 98.77) (width 0.2) (layer F.Cu) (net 18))
 (segment (start 236.31 113.2168) (end 236.31 99.972081) (width 0.2) (layer F.Cu) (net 18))
 (segment (start 235.4043 114.1225) (end 236.31 113.2168) (width 0.2) (layer F.Cu) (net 18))
 (segment (start 234.4043 114.1225) (end 235.4043 114.1225) (width 0.2) (layer F.Cu) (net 18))
 (segment (start 237.159999 97.079999) (end 236.31 96.23) (width 0.2) (layer F.Cu) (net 19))
 (segment (start 237.460001 97.380001) (end 237.159999 97.079999) (width 0.2) (layer F.Cu) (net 19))
 (segment (start 237.460001 112.701799) (end 237.460001 97.380001) (width 0.2) (layer F.Cu) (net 19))
 (segment (start 235.4043 114.7575) (end 237.460001 112.701799) (width 0.2) (layer F.Cu) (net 19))
 (segment (start 234.4043 114.7575) (end 235.4043 114.7575) (width 0.2) (layer F.Cu) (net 19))
 (segment (start 234.4043 112.2175) (end 234.4043 100.1017) (width 0.2) (layer F.Cu) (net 26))
 (segment (start 234.920001 99.585999) (end 234.920001 95.394999) (width 0.2) (layer F.Cu) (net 26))
 (segment (start 234.4043 100.1017) (end 234.920001 99.585999) (width 0.2) (layer F.Cu) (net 26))
 (segment (start 244.482001 95.079999) (end 245.212 95.809998) (width 0.2) (layer F.Cu) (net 26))
 (segment (start 235.235001 95.079999) (end 244.482001 95.079999) (width 0.2) (layer F.Cu) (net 26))
 (segment (start 234.920001 95.394999) (end 235.235001 95.079999) (width 0.2) (layer F.Cu) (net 26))
 (segment (start 248.160001 97.920001) (end 249.01 98.77) (width 0.2) (layer F.Cu) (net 26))
 (segment (start 247.859999 97.619999) (end 248.160001 97.920001) (width 0.2) (layer F.Cu) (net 26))
 (segment (start 246.171999 97.619999) (end 247.859999 97.619999) (width 0.2) (layer F.Cu) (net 26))
 (segment (start 245.212 96.66) (end 246.171999 97.619999) (width 0.2) (layer F.Cu) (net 26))
 (segment (start 245.212 95.809998) (end 245.212 96.66) (width 0.2) (layer F.Cu) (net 26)))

